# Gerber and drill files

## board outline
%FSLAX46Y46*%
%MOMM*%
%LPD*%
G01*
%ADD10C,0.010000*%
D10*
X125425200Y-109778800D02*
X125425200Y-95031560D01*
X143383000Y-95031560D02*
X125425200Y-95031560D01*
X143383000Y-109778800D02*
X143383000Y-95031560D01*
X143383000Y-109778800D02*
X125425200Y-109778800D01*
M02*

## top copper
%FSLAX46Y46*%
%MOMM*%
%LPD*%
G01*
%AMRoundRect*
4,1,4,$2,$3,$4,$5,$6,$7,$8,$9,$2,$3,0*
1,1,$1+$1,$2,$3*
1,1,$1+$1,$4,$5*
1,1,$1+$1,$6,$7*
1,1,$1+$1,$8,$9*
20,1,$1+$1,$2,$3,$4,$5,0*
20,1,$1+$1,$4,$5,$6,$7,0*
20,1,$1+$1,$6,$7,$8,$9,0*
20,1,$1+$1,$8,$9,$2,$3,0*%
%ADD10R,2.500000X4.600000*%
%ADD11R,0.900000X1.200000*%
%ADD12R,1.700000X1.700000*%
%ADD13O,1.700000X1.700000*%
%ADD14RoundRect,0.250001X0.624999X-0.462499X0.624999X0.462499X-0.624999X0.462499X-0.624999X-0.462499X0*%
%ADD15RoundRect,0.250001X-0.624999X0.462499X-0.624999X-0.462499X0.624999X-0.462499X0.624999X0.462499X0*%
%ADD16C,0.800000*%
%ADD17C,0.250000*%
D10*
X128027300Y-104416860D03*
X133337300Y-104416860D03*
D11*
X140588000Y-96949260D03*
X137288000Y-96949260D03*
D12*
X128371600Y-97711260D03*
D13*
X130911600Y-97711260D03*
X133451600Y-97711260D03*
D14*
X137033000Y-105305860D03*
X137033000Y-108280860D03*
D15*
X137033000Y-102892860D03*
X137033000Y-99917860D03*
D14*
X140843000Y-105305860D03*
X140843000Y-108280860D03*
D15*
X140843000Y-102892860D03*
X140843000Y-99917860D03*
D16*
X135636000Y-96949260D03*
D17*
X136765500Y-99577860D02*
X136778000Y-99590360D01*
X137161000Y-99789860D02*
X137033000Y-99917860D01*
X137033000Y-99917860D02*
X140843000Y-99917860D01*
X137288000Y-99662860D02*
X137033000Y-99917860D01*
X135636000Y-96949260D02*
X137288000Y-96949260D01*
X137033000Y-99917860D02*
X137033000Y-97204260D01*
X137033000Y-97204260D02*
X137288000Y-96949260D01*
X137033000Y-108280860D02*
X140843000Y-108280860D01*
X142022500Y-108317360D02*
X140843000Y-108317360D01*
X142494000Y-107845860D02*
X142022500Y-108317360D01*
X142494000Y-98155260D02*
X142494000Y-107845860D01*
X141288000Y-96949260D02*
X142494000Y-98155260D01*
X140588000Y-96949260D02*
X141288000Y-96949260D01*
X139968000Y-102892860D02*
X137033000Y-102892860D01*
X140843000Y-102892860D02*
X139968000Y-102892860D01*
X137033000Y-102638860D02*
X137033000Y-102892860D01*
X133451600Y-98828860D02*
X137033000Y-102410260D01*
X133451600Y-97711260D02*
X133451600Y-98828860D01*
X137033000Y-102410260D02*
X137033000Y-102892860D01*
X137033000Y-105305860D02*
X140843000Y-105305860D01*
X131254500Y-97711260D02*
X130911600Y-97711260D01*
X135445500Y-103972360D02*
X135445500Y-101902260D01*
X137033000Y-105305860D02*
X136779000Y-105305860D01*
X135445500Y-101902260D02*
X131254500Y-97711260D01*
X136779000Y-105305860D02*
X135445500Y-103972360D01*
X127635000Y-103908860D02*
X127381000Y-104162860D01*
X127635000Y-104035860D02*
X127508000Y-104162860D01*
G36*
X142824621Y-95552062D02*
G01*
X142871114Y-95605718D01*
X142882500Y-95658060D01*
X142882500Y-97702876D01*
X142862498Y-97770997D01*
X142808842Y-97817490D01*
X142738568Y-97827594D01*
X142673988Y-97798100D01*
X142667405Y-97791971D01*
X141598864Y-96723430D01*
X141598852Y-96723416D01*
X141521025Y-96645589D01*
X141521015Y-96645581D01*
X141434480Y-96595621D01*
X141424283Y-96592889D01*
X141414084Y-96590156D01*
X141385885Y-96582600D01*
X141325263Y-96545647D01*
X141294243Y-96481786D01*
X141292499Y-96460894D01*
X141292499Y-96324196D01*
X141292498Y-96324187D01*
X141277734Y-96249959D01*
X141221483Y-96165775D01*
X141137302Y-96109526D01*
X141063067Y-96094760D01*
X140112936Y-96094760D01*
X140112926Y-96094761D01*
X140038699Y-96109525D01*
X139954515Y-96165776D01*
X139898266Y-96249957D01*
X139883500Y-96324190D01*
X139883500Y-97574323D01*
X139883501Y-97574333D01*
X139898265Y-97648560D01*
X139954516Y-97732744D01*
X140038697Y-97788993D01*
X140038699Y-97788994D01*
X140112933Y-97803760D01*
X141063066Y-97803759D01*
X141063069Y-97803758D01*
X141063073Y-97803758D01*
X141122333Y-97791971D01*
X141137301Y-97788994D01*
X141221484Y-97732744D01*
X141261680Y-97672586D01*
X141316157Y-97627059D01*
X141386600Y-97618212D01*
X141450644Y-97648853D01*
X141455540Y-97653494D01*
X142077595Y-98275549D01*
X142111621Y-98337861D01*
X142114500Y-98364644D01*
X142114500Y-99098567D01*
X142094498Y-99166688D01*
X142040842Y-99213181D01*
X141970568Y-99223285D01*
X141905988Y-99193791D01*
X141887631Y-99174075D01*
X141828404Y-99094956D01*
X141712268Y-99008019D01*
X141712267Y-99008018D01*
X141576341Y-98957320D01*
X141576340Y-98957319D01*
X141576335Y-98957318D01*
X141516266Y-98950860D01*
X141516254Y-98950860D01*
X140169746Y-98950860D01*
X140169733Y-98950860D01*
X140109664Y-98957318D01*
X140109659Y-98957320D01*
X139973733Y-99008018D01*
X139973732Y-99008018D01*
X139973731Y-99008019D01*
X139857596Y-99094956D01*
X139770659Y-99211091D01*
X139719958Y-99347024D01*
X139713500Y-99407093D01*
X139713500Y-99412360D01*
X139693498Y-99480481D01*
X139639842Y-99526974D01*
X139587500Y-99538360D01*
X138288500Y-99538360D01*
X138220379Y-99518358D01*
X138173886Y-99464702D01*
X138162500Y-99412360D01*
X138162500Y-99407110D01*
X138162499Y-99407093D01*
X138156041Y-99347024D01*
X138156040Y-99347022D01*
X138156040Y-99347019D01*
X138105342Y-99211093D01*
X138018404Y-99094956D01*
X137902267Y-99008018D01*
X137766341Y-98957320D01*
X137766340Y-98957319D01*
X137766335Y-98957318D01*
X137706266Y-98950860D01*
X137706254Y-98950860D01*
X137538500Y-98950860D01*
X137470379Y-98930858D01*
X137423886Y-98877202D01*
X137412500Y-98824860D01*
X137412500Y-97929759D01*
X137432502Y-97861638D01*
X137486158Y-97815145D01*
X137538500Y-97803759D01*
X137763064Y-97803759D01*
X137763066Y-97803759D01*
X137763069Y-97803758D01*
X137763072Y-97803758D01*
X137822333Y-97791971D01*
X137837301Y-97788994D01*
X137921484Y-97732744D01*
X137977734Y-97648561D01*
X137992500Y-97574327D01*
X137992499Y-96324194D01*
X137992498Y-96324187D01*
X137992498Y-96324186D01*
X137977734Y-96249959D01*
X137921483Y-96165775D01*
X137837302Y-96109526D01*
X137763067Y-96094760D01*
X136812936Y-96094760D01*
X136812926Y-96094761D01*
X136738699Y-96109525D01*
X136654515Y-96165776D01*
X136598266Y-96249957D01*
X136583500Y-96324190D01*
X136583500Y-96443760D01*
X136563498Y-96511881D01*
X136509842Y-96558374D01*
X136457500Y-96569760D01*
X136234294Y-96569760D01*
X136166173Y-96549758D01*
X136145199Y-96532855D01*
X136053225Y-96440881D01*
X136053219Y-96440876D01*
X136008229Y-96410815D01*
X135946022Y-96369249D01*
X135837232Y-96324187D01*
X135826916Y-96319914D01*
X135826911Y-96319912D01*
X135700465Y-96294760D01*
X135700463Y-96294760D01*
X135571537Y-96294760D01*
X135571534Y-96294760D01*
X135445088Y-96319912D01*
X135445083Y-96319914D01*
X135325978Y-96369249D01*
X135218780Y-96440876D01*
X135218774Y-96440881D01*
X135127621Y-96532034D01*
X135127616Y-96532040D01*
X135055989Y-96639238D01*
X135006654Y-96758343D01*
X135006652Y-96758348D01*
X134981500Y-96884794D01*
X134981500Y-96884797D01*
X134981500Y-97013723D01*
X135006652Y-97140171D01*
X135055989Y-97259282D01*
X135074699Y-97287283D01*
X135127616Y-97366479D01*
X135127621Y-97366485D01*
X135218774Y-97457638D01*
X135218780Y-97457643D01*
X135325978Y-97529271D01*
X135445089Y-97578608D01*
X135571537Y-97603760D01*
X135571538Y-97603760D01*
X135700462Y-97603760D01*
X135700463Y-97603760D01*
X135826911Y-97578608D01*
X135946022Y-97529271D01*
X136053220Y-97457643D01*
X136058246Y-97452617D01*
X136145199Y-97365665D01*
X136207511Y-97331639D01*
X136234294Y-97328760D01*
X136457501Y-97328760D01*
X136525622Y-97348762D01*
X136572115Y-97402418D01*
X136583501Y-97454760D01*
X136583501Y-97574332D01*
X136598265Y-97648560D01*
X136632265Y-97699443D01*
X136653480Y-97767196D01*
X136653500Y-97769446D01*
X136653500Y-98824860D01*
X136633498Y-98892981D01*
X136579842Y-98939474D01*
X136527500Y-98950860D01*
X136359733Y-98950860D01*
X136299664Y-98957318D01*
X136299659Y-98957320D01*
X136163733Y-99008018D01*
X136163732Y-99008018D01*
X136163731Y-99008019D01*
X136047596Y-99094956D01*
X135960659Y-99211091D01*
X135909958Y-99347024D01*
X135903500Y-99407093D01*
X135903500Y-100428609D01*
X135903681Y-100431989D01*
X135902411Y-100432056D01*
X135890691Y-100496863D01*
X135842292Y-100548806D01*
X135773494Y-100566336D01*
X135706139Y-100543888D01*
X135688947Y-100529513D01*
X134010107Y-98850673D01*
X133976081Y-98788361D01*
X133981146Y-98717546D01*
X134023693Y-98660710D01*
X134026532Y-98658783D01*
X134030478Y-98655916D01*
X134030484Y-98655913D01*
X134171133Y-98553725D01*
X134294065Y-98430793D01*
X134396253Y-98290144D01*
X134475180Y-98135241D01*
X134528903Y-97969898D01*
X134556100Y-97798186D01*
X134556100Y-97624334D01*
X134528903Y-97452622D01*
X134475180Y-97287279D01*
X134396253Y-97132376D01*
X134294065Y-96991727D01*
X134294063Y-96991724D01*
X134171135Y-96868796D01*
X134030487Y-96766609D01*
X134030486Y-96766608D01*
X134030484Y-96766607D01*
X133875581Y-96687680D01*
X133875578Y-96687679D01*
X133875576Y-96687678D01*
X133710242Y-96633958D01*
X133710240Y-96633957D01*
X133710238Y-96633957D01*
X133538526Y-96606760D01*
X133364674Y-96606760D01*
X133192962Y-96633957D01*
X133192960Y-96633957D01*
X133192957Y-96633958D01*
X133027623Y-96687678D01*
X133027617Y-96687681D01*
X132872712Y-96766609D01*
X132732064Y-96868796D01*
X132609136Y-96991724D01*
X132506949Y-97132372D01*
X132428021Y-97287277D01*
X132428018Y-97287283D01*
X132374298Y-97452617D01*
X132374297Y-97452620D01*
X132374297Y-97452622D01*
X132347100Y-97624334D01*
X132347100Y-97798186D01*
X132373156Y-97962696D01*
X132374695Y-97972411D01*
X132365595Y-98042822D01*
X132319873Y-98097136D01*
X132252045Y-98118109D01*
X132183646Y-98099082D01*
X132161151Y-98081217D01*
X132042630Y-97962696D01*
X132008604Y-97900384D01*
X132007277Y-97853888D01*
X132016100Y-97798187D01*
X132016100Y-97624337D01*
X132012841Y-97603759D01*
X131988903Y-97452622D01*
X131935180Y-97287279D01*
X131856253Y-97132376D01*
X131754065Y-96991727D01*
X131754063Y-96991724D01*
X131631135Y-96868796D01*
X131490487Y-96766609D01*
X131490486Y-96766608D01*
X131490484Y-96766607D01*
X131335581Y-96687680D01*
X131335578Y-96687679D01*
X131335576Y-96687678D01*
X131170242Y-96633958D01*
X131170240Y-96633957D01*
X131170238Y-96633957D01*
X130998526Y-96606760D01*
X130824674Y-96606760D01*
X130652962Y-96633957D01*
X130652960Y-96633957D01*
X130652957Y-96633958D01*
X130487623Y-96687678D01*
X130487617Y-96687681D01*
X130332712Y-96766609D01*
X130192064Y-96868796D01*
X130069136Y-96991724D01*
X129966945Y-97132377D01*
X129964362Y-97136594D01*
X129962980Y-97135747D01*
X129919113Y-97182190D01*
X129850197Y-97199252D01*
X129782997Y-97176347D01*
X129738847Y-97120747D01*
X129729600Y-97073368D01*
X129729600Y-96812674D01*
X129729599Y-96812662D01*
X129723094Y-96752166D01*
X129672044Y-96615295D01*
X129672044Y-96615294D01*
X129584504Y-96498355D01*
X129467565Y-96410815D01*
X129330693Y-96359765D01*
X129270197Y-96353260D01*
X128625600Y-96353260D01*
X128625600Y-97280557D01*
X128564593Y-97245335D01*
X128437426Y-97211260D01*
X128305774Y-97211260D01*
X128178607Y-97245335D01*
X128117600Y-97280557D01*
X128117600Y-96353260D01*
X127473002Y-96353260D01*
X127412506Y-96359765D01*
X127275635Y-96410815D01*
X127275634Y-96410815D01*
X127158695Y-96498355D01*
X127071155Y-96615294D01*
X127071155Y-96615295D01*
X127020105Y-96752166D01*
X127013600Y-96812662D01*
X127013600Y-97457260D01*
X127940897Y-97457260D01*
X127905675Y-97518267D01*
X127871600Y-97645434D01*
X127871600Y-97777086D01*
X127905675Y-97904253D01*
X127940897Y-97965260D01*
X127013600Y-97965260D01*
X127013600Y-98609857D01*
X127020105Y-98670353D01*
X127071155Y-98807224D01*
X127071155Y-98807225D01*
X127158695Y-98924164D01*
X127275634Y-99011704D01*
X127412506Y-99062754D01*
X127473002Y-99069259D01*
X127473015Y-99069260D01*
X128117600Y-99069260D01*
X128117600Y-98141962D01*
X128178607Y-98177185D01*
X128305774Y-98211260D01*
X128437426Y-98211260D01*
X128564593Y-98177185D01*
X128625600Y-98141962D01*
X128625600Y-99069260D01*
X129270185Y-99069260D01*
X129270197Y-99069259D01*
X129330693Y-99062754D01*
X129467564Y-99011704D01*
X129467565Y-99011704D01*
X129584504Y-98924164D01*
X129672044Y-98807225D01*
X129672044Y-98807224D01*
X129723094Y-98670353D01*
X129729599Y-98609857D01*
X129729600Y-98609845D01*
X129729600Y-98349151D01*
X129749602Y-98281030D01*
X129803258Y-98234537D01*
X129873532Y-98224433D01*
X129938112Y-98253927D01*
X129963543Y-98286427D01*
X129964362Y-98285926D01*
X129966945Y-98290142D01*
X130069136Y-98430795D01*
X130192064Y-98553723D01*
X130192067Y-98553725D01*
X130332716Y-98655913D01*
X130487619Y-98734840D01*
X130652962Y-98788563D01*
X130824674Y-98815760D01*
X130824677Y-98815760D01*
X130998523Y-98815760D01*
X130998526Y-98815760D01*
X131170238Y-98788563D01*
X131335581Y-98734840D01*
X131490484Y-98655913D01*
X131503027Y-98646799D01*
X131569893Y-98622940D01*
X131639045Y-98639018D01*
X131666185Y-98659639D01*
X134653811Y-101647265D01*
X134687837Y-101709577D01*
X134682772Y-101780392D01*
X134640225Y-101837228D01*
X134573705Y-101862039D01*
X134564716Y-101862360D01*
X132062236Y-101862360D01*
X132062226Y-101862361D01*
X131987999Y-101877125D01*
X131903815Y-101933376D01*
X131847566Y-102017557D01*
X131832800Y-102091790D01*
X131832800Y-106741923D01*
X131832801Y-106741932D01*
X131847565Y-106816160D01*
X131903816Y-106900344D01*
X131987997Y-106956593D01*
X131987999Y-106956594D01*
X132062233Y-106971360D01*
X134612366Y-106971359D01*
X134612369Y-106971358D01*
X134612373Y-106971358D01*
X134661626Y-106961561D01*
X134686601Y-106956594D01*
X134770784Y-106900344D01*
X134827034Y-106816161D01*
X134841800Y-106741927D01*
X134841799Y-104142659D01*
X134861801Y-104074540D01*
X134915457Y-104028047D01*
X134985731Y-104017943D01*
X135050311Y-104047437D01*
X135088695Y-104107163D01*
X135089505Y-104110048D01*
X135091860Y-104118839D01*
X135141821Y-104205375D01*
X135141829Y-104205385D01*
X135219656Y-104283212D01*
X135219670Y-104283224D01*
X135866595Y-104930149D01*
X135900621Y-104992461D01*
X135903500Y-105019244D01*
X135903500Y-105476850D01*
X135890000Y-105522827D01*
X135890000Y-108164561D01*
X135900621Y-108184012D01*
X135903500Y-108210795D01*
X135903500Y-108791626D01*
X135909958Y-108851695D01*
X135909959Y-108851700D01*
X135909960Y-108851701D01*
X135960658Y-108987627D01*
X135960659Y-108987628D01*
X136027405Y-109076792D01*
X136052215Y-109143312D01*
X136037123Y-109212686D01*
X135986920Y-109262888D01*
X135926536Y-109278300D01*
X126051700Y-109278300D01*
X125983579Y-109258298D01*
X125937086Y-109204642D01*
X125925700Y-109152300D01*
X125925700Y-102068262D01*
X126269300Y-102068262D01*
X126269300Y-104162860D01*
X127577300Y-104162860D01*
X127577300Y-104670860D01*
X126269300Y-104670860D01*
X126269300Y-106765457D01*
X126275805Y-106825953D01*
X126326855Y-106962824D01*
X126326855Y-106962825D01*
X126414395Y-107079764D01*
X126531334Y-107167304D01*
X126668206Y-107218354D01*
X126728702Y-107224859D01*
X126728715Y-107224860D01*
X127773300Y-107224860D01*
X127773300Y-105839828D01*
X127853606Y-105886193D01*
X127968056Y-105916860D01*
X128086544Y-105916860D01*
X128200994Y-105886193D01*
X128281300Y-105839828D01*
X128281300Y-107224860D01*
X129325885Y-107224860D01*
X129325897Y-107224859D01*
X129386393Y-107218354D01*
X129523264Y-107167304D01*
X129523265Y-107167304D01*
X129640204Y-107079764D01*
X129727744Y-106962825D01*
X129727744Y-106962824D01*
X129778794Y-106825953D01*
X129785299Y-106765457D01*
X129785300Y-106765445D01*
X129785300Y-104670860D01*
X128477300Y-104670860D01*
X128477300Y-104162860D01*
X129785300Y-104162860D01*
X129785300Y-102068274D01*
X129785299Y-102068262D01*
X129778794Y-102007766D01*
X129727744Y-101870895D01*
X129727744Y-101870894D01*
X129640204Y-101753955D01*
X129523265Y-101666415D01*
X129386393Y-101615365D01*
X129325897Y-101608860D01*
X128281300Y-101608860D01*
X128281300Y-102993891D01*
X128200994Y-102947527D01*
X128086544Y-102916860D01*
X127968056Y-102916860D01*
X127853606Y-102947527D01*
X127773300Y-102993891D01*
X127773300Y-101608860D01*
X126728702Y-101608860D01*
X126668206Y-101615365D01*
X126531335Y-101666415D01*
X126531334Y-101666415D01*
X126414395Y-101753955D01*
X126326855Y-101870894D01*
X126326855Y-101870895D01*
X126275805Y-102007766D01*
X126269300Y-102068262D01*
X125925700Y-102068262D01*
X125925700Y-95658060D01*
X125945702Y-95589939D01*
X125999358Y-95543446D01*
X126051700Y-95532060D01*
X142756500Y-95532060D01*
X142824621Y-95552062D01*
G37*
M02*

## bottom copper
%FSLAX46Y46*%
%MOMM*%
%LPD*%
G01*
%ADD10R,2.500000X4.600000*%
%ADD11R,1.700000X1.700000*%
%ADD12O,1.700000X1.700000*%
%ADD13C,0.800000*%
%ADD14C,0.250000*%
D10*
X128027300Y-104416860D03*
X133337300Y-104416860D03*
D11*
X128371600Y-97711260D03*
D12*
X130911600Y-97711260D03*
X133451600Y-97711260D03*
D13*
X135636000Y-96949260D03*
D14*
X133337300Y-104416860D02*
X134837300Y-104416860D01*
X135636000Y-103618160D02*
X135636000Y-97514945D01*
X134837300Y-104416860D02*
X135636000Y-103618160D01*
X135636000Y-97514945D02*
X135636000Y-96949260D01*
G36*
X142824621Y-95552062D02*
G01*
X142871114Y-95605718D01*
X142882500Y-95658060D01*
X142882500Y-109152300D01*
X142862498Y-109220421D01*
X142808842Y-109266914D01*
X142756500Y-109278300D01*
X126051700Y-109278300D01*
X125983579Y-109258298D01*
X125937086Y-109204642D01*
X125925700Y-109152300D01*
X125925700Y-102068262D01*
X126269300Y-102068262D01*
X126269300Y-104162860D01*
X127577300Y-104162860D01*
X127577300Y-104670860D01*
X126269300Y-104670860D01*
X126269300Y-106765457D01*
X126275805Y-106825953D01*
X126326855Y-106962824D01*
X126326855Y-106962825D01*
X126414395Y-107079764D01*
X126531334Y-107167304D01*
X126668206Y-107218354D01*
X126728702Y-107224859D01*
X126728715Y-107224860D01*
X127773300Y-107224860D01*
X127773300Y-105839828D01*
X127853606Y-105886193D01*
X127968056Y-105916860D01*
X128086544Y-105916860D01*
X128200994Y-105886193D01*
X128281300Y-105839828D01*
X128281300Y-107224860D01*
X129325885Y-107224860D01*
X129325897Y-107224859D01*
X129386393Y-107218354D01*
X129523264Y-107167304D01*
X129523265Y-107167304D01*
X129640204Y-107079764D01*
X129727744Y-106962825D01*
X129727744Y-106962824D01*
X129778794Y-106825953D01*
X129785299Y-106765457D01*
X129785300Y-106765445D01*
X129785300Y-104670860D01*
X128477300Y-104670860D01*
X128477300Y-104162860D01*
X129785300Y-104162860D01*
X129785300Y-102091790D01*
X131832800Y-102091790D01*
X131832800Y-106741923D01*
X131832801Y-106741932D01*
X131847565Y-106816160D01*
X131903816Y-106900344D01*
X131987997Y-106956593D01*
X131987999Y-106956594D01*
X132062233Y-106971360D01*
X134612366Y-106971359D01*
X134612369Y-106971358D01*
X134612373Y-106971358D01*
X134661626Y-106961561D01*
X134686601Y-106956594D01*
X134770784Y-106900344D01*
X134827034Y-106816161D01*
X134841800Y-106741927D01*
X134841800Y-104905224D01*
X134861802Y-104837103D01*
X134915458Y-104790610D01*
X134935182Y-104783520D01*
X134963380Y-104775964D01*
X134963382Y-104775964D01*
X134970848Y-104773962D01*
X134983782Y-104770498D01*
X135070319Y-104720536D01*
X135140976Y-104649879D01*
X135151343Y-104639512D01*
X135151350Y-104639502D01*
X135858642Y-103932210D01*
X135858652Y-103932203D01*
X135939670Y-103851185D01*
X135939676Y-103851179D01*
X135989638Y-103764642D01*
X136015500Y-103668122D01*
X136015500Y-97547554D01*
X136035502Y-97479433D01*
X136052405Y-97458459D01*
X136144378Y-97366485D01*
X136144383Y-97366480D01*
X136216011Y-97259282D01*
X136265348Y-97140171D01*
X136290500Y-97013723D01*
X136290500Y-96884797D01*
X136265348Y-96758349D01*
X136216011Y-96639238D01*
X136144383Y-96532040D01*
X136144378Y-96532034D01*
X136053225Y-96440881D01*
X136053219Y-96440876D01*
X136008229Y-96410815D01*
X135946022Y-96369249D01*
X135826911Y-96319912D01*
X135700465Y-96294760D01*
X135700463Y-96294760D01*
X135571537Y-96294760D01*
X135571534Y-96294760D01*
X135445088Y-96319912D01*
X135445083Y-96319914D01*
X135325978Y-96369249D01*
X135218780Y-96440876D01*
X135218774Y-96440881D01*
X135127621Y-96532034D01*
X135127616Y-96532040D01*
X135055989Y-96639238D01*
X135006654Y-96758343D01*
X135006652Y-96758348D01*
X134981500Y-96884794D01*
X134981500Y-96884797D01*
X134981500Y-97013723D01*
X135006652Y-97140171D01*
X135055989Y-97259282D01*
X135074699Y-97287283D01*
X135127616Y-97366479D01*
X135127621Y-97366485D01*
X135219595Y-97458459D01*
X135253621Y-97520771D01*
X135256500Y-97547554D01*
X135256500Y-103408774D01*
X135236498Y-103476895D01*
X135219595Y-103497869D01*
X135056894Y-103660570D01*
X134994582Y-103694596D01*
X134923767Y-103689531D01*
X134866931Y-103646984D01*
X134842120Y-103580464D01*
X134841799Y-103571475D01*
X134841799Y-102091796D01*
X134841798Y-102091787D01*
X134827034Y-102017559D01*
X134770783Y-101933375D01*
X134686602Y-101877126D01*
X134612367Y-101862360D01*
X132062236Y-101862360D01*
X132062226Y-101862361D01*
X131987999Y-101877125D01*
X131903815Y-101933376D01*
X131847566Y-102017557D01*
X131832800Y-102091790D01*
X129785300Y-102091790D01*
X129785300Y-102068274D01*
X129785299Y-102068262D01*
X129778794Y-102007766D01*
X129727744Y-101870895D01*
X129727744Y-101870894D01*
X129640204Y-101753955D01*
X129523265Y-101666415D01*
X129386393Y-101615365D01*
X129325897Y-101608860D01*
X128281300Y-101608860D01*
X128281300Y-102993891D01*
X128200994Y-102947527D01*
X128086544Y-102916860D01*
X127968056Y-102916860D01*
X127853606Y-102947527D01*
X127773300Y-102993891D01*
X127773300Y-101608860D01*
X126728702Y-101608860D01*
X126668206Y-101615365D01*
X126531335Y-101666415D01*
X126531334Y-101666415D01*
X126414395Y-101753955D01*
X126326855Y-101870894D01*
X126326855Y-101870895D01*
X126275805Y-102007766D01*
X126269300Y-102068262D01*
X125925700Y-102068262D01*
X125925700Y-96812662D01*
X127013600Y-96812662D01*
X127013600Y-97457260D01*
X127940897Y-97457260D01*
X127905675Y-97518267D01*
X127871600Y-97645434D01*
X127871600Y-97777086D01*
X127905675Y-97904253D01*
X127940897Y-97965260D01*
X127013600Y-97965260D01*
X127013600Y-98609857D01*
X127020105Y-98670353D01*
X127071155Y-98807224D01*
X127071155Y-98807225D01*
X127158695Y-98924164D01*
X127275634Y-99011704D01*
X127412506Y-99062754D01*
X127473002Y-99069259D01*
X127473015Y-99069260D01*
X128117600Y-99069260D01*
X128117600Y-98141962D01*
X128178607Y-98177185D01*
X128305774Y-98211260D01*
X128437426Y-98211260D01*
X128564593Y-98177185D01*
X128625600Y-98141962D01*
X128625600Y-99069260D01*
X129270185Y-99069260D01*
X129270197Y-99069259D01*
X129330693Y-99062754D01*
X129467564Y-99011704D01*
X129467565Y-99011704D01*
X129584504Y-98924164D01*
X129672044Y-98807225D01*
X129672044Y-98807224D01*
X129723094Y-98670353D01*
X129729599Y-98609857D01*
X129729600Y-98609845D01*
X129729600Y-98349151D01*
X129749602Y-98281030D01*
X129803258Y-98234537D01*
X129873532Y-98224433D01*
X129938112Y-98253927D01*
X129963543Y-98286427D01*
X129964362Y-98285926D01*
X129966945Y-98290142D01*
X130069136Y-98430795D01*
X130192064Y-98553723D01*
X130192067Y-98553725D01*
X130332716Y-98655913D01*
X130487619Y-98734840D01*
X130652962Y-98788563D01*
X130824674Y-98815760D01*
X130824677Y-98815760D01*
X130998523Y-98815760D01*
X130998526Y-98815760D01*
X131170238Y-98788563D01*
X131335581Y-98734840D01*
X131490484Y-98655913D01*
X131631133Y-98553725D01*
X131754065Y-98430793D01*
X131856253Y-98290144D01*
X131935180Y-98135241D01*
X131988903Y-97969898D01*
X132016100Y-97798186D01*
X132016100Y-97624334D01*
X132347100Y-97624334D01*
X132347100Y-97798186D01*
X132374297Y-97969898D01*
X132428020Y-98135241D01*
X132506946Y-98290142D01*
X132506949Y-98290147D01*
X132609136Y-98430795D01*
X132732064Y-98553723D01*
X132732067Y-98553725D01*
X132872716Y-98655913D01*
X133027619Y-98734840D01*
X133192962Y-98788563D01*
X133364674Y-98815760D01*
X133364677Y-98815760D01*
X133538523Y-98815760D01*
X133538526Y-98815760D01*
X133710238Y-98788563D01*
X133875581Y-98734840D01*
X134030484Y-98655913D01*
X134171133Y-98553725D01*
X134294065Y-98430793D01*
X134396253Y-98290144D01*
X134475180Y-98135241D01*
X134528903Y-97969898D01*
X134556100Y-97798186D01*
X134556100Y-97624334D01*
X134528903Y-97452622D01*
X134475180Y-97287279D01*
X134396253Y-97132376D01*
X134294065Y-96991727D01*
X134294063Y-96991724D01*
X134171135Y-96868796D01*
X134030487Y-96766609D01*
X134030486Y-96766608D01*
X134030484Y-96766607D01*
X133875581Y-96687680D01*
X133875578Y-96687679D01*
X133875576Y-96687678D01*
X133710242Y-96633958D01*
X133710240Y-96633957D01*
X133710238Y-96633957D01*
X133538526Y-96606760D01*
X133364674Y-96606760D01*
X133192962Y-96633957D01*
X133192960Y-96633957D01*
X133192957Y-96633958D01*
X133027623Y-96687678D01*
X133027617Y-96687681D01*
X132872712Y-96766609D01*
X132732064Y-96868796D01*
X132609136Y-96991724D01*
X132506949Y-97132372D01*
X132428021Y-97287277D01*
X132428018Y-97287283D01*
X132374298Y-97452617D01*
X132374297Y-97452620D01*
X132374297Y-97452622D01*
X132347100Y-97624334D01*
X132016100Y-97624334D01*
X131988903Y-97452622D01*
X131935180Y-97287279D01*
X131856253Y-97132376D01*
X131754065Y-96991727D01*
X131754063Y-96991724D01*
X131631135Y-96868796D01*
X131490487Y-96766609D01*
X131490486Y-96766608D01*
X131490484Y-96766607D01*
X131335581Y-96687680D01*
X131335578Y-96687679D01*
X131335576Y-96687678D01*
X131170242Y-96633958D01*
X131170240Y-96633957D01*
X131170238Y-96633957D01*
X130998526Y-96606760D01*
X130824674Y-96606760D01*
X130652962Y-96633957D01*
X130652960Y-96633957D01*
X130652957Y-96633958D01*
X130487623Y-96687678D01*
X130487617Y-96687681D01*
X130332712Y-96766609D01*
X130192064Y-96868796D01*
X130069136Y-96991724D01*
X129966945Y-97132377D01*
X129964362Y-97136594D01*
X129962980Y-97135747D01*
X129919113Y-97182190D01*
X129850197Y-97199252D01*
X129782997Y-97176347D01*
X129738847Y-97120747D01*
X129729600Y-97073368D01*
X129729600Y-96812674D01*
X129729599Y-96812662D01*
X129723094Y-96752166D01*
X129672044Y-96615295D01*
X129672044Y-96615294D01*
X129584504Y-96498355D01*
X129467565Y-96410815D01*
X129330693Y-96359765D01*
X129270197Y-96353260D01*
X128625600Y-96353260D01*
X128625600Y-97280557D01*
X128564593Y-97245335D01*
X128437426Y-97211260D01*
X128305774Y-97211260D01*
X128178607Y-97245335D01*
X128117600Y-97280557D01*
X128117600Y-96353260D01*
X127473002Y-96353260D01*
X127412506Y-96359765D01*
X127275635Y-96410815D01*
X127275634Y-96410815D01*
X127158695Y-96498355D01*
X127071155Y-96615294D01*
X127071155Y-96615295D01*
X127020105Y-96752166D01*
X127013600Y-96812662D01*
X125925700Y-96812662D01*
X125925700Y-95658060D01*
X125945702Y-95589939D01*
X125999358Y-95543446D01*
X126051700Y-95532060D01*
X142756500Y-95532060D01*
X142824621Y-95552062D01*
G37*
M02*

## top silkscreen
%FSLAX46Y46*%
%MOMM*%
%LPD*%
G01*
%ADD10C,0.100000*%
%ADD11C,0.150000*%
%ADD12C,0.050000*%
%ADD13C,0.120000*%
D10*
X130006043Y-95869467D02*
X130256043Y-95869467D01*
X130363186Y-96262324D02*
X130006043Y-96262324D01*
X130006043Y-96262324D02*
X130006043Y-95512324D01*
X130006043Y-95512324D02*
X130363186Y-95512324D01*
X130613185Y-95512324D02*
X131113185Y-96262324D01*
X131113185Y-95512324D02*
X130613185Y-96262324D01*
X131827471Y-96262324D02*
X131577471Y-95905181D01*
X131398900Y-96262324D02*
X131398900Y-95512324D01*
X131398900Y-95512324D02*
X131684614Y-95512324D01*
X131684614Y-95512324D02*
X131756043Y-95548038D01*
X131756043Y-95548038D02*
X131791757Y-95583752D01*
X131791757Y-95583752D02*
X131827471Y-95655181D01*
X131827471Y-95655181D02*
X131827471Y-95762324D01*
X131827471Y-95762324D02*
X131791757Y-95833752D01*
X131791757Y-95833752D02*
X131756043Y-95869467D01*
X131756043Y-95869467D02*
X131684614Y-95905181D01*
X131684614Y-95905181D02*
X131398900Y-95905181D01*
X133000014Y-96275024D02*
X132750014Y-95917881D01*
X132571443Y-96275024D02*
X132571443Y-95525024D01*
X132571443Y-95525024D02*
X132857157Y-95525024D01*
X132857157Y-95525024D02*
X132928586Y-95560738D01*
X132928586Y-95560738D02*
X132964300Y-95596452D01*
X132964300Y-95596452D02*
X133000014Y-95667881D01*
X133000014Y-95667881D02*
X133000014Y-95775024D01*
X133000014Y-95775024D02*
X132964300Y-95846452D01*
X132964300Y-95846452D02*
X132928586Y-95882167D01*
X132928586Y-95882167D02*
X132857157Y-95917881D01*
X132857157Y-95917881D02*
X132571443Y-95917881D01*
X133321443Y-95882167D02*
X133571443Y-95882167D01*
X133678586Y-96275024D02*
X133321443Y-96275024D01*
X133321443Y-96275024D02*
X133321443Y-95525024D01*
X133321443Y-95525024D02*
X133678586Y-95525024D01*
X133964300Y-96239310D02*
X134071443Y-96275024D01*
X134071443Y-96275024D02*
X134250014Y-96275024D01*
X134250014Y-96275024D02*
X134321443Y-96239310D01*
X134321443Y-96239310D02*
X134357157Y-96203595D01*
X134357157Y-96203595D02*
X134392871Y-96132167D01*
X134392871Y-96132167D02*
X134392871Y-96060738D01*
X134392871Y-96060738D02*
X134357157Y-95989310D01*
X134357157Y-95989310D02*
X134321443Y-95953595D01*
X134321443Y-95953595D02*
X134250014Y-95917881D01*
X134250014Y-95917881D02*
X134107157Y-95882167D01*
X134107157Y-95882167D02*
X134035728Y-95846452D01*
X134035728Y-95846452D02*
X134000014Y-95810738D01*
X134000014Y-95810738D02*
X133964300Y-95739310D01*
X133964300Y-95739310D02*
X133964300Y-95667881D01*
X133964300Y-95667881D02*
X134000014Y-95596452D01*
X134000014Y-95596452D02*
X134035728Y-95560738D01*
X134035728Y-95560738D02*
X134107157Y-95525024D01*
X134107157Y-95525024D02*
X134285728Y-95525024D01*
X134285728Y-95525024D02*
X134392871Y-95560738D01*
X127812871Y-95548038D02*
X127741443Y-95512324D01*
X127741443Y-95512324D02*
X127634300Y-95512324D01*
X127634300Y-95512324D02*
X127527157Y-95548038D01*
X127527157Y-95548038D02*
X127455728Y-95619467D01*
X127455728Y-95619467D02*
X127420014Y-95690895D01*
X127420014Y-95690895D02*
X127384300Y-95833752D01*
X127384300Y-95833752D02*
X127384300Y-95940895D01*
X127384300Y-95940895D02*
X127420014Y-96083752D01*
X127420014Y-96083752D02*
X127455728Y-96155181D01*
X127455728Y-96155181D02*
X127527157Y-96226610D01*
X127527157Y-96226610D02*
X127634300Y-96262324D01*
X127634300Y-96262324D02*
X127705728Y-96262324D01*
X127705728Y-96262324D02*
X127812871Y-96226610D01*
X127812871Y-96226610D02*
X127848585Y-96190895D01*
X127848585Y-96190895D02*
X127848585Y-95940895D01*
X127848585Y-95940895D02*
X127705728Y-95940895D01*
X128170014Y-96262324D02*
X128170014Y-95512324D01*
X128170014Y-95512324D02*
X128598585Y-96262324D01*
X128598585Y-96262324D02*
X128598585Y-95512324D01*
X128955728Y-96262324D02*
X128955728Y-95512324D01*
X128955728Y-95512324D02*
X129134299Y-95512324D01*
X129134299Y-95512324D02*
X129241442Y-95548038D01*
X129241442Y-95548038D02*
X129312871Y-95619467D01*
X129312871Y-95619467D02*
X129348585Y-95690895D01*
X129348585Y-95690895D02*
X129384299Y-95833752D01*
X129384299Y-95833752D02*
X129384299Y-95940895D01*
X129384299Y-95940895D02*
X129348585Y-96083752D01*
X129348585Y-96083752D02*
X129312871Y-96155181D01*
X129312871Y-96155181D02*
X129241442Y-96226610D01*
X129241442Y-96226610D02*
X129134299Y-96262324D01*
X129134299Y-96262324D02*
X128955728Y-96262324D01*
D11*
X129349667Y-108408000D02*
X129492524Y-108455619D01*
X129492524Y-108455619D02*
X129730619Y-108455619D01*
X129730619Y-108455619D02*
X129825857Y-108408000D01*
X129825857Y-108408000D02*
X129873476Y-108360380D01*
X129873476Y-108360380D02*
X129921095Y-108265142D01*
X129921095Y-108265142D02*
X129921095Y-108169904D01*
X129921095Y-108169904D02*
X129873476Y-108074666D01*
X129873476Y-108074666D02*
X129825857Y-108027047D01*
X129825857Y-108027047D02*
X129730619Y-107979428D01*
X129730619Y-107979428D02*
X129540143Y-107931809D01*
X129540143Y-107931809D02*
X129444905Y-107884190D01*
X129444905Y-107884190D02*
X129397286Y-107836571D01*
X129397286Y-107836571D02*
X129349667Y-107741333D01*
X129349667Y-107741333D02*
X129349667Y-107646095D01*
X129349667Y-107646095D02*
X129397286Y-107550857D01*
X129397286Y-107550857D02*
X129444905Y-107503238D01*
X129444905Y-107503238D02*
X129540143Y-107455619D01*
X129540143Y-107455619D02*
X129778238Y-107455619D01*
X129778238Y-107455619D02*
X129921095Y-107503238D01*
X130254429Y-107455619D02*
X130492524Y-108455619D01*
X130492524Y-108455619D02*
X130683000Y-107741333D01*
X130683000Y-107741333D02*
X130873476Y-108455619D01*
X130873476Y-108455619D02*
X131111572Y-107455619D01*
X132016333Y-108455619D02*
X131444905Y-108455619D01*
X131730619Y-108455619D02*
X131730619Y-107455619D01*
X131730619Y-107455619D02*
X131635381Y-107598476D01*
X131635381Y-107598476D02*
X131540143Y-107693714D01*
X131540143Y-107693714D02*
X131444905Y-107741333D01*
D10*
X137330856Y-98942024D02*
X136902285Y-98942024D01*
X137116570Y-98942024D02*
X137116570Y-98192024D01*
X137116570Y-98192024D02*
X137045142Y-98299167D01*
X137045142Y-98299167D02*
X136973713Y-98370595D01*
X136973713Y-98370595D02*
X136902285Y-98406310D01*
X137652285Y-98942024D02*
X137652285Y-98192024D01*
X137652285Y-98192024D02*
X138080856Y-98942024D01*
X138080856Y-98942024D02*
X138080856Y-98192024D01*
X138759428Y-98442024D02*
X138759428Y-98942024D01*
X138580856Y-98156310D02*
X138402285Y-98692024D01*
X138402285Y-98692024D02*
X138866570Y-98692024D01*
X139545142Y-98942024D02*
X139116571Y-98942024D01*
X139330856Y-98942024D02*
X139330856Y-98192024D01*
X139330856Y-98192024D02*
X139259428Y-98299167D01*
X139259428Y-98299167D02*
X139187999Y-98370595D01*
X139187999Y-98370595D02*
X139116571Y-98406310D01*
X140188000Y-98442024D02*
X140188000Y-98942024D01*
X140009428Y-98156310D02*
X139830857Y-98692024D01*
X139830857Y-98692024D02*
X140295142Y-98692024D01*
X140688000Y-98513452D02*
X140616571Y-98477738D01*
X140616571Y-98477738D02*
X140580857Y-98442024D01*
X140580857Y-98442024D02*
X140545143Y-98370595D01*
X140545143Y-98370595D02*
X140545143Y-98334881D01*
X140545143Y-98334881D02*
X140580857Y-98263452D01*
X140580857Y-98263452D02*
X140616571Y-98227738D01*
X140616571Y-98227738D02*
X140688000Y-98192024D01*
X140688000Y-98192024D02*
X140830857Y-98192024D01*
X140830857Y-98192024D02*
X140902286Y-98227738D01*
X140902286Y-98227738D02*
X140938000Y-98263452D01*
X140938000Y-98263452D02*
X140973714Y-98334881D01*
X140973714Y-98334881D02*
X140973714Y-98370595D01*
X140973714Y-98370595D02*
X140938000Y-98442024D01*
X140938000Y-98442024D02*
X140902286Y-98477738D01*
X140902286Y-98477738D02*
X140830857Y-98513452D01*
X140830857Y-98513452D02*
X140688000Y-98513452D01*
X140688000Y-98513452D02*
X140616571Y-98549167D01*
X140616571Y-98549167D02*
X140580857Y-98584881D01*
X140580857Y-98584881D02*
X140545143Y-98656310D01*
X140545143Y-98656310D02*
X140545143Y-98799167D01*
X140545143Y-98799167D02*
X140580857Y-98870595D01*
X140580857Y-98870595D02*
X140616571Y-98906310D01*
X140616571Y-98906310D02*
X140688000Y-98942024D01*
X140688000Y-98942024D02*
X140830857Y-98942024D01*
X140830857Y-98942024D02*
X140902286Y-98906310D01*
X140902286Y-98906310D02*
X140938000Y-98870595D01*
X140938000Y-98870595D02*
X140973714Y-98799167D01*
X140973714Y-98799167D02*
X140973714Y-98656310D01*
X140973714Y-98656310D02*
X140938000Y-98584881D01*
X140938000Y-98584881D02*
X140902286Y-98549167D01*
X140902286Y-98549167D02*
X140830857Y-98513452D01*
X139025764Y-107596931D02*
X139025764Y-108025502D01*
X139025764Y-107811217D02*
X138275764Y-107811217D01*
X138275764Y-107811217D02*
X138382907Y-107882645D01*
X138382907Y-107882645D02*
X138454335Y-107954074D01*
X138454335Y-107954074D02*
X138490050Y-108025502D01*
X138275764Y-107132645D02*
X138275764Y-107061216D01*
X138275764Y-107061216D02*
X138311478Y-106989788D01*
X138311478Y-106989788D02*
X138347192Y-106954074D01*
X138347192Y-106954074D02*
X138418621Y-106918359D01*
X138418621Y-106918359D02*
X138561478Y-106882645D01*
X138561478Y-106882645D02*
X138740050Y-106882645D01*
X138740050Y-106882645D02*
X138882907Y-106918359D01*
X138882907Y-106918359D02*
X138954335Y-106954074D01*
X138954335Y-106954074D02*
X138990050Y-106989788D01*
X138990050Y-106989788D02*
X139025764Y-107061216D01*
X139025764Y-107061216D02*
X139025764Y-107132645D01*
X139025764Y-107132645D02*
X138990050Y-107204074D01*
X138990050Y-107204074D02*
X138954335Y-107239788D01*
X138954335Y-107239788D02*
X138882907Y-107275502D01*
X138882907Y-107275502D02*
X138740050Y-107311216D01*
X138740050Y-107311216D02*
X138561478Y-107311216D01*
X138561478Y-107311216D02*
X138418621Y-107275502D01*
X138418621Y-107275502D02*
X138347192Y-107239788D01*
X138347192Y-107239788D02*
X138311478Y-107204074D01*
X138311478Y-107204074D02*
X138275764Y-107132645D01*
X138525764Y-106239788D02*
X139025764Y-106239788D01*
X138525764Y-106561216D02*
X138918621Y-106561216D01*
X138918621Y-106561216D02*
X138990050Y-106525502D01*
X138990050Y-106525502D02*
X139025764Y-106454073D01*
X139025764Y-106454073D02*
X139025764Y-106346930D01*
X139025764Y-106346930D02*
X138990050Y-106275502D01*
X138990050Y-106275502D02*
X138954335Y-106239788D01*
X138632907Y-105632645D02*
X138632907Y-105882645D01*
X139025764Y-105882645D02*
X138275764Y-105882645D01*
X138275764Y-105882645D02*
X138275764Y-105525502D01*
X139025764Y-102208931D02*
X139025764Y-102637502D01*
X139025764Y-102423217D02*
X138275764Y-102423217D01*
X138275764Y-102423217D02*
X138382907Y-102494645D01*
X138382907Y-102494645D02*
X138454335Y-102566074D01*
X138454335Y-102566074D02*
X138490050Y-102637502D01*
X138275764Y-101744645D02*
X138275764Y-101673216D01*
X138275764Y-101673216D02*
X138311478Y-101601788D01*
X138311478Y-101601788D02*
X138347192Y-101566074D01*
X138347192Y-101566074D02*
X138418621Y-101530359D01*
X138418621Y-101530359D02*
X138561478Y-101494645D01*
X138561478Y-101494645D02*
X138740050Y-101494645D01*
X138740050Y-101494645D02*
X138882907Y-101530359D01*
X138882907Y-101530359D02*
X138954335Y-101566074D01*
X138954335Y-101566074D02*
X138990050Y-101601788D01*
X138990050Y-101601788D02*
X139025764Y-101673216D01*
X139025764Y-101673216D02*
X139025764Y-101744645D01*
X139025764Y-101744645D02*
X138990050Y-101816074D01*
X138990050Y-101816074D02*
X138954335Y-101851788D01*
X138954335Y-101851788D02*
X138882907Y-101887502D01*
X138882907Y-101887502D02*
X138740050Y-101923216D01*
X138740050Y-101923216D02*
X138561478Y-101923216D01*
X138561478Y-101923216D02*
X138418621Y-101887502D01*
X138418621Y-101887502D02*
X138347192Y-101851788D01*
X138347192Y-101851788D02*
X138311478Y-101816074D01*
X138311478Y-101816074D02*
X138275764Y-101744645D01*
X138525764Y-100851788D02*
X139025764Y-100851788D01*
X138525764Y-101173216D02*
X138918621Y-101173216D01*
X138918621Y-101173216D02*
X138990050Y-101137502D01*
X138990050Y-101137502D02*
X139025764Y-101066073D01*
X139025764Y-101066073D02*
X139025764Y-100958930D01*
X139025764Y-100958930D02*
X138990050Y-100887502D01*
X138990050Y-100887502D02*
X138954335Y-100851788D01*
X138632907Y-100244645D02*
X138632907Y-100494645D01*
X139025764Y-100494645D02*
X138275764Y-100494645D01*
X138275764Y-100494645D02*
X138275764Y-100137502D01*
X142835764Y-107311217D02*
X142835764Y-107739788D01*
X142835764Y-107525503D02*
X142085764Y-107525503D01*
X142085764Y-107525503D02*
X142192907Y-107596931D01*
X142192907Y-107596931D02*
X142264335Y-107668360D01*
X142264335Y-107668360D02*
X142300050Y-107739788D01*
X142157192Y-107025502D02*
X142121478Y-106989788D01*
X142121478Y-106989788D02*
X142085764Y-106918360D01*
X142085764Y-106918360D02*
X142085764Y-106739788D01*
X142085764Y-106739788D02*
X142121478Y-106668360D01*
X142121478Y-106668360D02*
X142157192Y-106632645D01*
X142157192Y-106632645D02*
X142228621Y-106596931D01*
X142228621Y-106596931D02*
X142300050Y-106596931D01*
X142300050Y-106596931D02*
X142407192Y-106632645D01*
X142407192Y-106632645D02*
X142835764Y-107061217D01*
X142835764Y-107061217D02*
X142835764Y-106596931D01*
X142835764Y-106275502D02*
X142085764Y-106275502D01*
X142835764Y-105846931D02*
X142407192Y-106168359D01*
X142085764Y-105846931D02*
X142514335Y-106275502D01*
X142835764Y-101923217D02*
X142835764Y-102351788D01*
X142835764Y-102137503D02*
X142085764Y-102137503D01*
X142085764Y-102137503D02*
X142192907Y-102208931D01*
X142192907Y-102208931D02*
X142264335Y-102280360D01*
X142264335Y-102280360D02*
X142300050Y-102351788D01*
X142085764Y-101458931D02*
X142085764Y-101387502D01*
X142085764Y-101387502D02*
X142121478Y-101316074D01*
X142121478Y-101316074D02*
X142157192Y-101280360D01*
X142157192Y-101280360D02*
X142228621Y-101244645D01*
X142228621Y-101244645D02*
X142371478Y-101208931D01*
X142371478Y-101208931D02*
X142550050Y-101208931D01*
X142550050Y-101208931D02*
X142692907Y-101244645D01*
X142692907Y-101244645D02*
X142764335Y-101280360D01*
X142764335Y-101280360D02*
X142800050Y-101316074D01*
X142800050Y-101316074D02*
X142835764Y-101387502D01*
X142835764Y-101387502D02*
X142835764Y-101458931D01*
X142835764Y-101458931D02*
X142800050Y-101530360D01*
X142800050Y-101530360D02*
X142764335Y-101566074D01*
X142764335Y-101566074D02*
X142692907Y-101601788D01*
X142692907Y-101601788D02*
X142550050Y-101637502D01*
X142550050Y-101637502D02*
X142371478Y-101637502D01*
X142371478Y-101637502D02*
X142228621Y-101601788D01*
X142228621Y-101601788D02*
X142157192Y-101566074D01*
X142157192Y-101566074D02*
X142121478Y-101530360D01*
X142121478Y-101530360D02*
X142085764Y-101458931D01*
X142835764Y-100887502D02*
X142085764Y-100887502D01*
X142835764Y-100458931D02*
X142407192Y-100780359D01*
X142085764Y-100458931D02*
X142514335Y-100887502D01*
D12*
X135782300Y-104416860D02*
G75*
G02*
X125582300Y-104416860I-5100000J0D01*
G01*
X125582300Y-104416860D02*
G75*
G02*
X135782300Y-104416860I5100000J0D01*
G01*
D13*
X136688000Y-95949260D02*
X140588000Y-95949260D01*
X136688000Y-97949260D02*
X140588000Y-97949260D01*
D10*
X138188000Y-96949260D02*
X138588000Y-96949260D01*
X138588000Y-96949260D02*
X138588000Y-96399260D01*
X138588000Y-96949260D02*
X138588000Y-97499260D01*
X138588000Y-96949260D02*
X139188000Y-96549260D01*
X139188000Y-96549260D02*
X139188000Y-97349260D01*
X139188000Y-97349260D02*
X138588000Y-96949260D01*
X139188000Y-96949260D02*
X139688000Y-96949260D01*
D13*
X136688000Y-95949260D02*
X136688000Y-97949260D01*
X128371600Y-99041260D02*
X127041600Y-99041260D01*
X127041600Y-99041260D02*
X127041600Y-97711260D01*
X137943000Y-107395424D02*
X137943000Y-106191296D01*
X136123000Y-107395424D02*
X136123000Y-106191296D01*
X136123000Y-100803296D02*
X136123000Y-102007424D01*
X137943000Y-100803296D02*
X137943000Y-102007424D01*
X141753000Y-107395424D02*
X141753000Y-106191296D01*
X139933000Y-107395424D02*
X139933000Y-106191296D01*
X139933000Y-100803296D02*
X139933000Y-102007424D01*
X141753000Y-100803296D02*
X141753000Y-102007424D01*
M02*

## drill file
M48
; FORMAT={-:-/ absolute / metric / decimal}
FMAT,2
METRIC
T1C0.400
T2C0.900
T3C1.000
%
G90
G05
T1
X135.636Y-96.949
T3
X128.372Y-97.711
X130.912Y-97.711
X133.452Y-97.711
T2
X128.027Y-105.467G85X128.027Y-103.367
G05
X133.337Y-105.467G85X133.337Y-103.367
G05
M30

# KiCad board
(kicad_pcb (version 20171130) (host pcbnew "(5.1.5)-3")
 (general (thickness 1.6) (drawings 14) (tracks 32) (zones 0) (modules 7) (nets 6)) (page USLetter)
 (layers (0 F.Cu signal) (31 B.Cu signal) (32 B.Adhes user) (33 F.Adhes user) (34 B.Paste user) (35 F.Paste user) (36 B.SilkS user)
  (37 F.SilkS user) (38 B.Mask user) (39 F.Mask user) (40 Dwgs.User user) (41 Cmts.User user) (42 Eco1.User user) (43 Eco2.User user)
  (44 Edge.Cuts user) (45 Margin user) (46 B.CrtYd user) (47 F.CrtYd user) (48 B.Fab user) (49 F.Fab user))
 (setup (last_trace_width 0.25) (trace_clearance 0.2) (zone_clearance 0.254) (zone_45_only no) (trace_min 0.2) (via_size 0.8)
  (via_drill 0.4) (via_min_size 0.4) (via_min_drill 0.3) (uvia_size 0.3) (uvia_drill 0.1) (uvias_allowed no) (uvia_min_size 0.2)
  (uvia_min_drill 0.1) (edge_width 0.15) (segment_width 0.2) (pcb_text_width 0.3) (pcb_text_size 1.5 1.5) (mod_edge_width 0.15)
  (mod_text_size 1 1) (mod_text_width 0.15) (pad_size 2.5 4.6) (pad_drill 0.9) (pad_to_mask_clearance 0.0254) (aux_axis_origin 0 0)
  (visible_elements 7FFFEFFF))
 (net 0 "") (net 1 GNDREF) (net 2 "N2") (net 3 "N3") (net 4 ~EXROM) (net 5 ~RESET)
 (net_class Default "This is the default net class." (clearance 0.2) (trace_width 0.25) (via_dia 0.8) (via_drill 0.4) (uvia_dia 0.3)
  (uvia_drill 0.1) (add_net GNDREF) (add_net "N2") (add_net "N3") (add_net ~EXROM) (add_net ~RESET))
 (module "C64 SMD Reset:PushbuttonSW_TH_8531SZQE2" (layer F.Cu) (at 133.3373 104.41686 180)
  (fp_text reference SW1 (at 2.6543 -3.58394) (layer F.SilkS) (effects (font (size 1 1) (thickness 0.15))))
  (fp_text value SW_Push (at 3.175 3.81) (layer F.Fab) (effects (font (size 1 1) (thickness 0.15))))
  (fp_circle (center 2.655 0) (end 7.755 0) (layer F.SilkS) (width 0.05))
  (pad 2 thru_hole rect (at 5.31 0 180) (size 2.5 4.6) (drill oval 0.9 3) (layers *.Cu *.Mask) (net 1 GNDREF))
  (pad 1 thru_hole rect (at 0 0 180) (size 2.5 4.6) (drill oval 0.9 3) (layers *.Cu *.Mask) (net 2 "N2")))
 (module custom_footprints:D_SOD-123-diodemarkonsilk (layer F.Cu) (at 138.938 96.94926)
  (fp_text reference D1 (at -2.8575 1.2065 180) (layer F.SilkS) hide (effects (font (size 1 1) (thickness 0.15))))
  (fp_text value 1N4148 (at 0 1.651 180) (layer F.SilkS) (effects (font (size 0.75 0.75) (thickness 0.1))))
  (fp_line (start -2.25 -1) (end 1.65 -1) (layer F.SilkS) (width 0.12))
  (fp_line (start -2.25 1) (end 1.65 1) (layer F.SilkS) (width 0.12))
  (fp_line (start -0.75 0) (end -0.35 0) (layer F.SilkS) (width 0.1))
  (fp_line (start -0.35 0) (end -0.35 -0.55) (layer F.SilkS) (width 0.1))
  (fp_line (start -0.35 0) (end -0.35 0.55) (layer F.SilkS) (width 0.1))
  (fp_line (start -0.35 0) (end 0.25 -0.4) (layer F.SilkS) (width 0.1))
  (fp_line (start 0.25 -0.4) (end 0.25 0.4) (layer F.SilkS) (width 0.1))
  (fp_line (start 0.25 0.4) (end -0.35 0) (layer F.SilkS) (width 0.1))
  (fp_line (start 0.25 0) (end 0.75 0) (layer F.SilkS) (width 0.1))
  (fp_line (start -2.25 -1) (end -2.25 1) (layer F.SilkS) (width 0.12))
  (pad 2 smd rect (at 1.65 0) (size 0.9 1.2) (layers F.Cu F.Paste F.Mask) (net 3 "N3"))
  (pad 1 smd rect (at -1.65 0) (size 0.9 1.2) (layers F.Cu F.Paste F.Mask) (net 2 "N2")))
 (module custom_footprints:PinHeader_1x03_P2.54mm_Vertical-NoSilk (layer F.Cu) (at 128.3716 97.71126 90)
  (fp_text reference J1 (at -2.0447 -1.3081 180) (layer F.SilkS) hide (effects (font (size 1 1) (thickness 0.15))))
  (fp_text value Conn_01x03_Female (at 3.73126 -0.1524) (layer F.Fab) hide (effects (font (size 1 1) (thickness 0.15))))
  (fp_line (start -1.33 0) (end -1.33 -1.33) (layer F.SilkS) (width 0.12))
  (fp_line (start -1.33 -1.33) (end 0 -1.33) (layer F.SilkS) (width 0.12))
  (pad 1 thru_hole rect (at 0 0 90) (size 1.7 1.7) (drill 1) (layers *.Cu *.Mask) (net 1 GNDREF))
  (pad 2 thru_hole oval (at 0 2.54 90) (size 1.7 1.7) (drill 1) (layers *.Cu *.Mask) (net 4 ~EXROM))
  (pad 3 thru_hole oval (at 0 5.08 90) (size 1.7 1.7) (drill 1) (layers *.Cu *.Mask) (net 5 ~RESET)))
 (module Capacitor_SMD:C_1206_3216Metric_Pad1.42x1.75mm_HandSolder (layer F.Cu) (at 137.033 106.79336 90)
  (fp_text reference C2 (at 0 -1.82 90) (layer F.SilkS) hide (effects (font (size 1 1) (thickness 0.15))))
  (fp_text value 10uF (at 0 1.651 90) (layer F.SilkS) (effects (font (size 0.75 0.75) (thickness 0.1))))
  (fp_line (start -0.602064 0.91) (end 0.602064 0.91) (layer F.SilkS) (width 0.12))
  (fp_line (start -0.602064 -0.91) (end 0.602064 -0.91) (layer F.SilkS) (width 0.12))
  (pad 2 smd roundrect (at 1.4875 0 90) (size 1.425 1.75) (layers F.Cu F.Paste F.Mask) (roundrect_rratio 0.175439) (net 4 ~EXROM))
  (pad 1 smd roundrect (at -1.4875 0 90) (size 1.425 1.75) (layers F.Cu F.Paste F.Mask) (roundrect_rratio 0.175439) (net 3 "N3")))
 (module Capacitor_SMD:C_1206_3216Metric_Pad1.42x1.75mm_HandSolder (layer F.Cu) (at 137.033 101.40536 270)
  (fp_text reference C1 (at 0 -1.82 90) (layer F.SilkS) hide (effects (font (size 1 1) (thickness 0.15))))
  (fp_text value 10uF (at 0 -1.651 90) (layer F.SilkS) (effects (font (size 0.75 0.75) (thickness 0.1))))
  (fp_line (start -0.602064 0.91) (end 0.602064 0.91) (layer F.SilkS) (width 0.12))
  (fp_line (start -0.602064 -0.91) (end 0.602064 -0.91) (layer F.SilkS) (width 0.12))
  (pad 2 smd roundrect (at 1.4875 0 270) (size 1.425 1.75) (layers F.Cu F.Paste F.Mask) (roundrect_rratio 0.175439) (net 5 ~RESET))
  (pad 1 smd roundrect (at -1.4875 0 270) (size 1.425 1.75) (layers F.Cu F.Paste F.Mask) (roundrect_rratio 0.175439) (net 2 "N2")))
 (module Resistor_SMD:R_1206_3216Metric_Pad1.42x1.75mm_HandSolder (layer F.Cu) (at 140.843 106.79336 90)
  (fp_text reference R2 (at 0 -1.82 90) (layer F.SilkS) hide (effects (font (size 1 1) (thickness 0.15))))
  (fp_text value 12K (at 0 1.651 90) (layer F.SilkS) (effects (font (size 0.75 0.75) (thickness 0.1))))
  (fp_line (start -0.602064 0.91) (end 0.602064 0.91) (layer F.SilkS) (width 0.12))
  (fp_line (start -0.602064 -0.91) (end 0.602064 -0.91) (layer F.SilkS) (width 0.12))
  (pad 2 smd roundrect (at 1.4875 0 90) (size 1.425 1.75) (layers F.Cu F.Paste F.Mask) (roundrect_rratio 0.175439) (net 4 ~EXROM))
  (pad 1 smd roundrect (at -1.4875 0 90) (size 1.425 1.75) (layers F.Cu F.Paste F.Mask) (roundrect_rratio 0.175439) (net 3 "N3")))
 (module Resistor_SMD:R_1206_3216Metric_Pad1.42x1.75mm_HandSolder (layer F.Cu) (at 140.843 101.40536 270)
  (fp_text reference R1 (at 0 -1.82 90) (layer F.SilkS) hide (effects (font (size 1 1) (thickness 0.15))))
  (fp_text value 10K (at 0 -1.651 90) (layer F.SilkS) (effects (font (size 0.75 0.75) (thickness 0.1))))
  (fp_line (start -0.602064 0.91) (end 0.602064 0.91) (layer F.SilkS) (width 0.12))
  (fp_line (start -0.602064 -0.91) (end 0.602064 -0.91) (layer F.SilkS) (width 0.12))
  (pad 2 smd roundrect (at 1.4875 0 270) (size 1.425 1.75) (layers F.Cu F.Paste F.Mask) (roundrect_rratio 0.175439) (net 5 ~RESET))
  (pad 1 smd roundrect (at -1.4875 0 270) (size 1.425 1.75) (layers F.Cu F.Paste F.Mask) (roundrect_rratio 0.175439) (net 2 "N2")))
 (gr_line (start 125.4252 109.7788) (end 125.4252 95.03156) (layer Edge.Cuts) (width 0.01))
 (gr_line (start 143.383 95.03156) (end 125.4252 95.03156) (layer Edge.Cuts) (width 0.01))
 (gr_line (start 143.383 109.7788) (end 143.383 95.03156) (layer Edge.Cuts) (width 0.01))
 (gr_line (start 143.383 109.7788) (end 125.4252 109.7788) (layer Edge.Cuts) (width 0.01))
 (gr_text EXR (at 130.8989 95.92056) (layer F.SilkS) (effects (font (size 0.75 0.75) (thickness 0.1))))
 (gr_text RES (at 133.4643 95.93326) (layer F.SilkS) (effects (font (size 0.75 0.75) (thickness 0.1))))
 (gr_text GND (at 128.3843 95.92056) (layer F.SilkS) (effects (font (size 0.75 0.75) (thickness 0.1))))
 (segment (start 136.7655 99.57786) (end 136.778 99.59036) (width 0.25) (layer F.Cu) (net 2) (status 30))
 (segment (start 137.161 99.78986) (end 137.033 99.91786) (width 0.25) (layer F.Cu) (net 2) (status 30))
 (segment (start 137.033 99.91786) (end 140.843 99.91786) (width 0.25) (layer F.Cu) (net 2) (status 30))
 (segment (start 137.288 99.66286) (end 137.033 99.91786) (width 0.25) (layer F.Cu) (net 2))
 (segment (start 133.3373 104.41686) (end 134.8373 104.41686) (width 0.25) (layer B.Cu) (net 2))
 (segment (start 135.636 103.61816) (end 135.636 97.514945) (width 0.25) (layer B.Cu) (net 2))
 (via (at 135.636 96.94926) (size 0.8) (drill 0.4) (layers F.Cu B.Cu) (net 2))
 (segment (start 134.8373 104.41686) (end 135.636 103.61816) (width 0.25) (layer B.Cu) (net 2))
 (segment (start 135.636 97.514945) (end 135.636 96.94926) (width 0.25) (layer B.Cu) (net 2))
 (segment (start 135.636 96.94926) (end 137.288 96.94926) (width 0.25) (layer F.Cu) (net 2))
 (segment (start 137.033 99.91786) (end 137.033 97.20426) (width 0.25) (layer F.Cu) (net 2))
 (segment (start 137.033 97.20426) (end 137.288 96.94926) (width 0.25) (layer F.Cu) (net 2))
 (segment (start 137.033 108.28086) (end 140.843 108.28086) (width 0.25) (layer F.Cu) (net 3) (status 30))
 (segment (start 142.0225 108.31736) (end 140.843 108.31736) (width 0.25) (layer F.Cu) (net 3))
 (segment (start 142.494 107.84586) (end 142.0225 108.31736) (width 0.25) (layer F.Cu) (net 3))
 (segment (start 142.494 98.15526) (end 142.494 107.84586) (width 0.25) (layer F.Cu) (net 3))
 (segment (start 141.288 96.94926) (end 142.494 98.15526) (width 0.25) (layer F.Cu) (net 3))
 (segment (start 140.588 96.94926) (end 141.288 96.94926) (width 0.25) (layer F.Cu) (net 3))
 (segment (start 139.968 102.89286) (end 137.033 102.89286) (width 0.25) (layer F.Cu) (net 5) (status 30))
 (segment (start 140.843 102.89286) (end 139.968 102.89286) (width 0.25) (layer F.Cu) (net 5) (status 30))
 (segment (start 137.033 102.63886) (end 137.033 102.89286) (width 0.25) (layer F.Cu) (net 5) (status 30))
 (segment (start 133.4516 98.82886) (end 137.033 102.41026) (width 0.25) (layer F.Cu) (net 5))
 (segment (start 133.4516 97.71126) (end 133.4516 98.82886) (width 0.25) (layer F.Cu) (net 5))
 (segment (start 137.033 102.41026) (end 137.033 102.89286) (width 0.25) (layer F.Cu) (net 5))
 (segment (start 137.033 105.30586) (end 140.843 105.30586) (width 0.25) (layer F.Cu) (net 4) (status 30))
 (segment (start 131.2545 97.71126) (end 130.9116 97.71126) (width 0.25) (layer F.Cu) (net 4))
 (segment (start 135.4455 103.97236) (end 135.4455 101.90226) (width 0.25) (layer F.Cu) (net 4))
 (segment (start 137.033 105.30586) (end 136.779 105.30586) (width 0.25) (layer F.Cu) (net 4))
 (segment (start 135.4455 101.90226) (end 131.2545 97.71126) (width 0.25) (layer F.Cu) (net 4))
 (segment (start 136.779 105.30586) (end 135.4455 103.97236) (width 0.25) (layer F.Cu) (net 4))
 (segment (start 127.635 103.90886) (end 127.381 104.16286) (width 0.25) (layer F.Cu) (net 1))
 (segment (start 127.635 104.03586) (end 127.508 104.16286) (width 0.25) (layer F.Cu) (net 1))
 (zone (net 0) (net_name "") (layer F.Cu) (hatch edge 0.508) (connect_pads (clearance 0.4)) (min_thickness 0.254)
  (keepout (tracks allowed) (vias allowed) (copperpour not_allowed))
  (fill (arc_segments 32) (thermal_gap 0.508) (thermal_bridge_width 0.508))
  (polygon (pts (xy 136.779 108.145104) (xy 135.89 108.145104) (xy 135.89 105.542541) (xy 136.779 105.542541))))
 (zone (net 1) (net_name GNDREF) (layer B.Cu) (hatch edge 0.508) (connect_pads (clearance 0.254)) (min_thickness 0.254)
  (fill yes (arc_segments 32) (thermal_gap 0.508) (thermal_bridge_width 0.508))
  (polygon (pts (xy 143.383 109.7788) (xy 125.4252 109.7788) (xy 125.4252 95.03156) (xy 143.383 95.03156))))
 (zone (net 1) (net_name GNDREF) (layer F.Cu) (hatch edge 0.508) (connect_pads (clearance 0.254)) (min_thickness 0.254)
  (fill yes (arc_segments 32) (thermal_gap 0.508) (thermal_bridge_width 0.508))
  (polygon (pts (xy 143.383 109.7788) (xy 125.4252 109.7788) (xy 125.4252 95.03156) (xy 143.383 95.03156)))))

